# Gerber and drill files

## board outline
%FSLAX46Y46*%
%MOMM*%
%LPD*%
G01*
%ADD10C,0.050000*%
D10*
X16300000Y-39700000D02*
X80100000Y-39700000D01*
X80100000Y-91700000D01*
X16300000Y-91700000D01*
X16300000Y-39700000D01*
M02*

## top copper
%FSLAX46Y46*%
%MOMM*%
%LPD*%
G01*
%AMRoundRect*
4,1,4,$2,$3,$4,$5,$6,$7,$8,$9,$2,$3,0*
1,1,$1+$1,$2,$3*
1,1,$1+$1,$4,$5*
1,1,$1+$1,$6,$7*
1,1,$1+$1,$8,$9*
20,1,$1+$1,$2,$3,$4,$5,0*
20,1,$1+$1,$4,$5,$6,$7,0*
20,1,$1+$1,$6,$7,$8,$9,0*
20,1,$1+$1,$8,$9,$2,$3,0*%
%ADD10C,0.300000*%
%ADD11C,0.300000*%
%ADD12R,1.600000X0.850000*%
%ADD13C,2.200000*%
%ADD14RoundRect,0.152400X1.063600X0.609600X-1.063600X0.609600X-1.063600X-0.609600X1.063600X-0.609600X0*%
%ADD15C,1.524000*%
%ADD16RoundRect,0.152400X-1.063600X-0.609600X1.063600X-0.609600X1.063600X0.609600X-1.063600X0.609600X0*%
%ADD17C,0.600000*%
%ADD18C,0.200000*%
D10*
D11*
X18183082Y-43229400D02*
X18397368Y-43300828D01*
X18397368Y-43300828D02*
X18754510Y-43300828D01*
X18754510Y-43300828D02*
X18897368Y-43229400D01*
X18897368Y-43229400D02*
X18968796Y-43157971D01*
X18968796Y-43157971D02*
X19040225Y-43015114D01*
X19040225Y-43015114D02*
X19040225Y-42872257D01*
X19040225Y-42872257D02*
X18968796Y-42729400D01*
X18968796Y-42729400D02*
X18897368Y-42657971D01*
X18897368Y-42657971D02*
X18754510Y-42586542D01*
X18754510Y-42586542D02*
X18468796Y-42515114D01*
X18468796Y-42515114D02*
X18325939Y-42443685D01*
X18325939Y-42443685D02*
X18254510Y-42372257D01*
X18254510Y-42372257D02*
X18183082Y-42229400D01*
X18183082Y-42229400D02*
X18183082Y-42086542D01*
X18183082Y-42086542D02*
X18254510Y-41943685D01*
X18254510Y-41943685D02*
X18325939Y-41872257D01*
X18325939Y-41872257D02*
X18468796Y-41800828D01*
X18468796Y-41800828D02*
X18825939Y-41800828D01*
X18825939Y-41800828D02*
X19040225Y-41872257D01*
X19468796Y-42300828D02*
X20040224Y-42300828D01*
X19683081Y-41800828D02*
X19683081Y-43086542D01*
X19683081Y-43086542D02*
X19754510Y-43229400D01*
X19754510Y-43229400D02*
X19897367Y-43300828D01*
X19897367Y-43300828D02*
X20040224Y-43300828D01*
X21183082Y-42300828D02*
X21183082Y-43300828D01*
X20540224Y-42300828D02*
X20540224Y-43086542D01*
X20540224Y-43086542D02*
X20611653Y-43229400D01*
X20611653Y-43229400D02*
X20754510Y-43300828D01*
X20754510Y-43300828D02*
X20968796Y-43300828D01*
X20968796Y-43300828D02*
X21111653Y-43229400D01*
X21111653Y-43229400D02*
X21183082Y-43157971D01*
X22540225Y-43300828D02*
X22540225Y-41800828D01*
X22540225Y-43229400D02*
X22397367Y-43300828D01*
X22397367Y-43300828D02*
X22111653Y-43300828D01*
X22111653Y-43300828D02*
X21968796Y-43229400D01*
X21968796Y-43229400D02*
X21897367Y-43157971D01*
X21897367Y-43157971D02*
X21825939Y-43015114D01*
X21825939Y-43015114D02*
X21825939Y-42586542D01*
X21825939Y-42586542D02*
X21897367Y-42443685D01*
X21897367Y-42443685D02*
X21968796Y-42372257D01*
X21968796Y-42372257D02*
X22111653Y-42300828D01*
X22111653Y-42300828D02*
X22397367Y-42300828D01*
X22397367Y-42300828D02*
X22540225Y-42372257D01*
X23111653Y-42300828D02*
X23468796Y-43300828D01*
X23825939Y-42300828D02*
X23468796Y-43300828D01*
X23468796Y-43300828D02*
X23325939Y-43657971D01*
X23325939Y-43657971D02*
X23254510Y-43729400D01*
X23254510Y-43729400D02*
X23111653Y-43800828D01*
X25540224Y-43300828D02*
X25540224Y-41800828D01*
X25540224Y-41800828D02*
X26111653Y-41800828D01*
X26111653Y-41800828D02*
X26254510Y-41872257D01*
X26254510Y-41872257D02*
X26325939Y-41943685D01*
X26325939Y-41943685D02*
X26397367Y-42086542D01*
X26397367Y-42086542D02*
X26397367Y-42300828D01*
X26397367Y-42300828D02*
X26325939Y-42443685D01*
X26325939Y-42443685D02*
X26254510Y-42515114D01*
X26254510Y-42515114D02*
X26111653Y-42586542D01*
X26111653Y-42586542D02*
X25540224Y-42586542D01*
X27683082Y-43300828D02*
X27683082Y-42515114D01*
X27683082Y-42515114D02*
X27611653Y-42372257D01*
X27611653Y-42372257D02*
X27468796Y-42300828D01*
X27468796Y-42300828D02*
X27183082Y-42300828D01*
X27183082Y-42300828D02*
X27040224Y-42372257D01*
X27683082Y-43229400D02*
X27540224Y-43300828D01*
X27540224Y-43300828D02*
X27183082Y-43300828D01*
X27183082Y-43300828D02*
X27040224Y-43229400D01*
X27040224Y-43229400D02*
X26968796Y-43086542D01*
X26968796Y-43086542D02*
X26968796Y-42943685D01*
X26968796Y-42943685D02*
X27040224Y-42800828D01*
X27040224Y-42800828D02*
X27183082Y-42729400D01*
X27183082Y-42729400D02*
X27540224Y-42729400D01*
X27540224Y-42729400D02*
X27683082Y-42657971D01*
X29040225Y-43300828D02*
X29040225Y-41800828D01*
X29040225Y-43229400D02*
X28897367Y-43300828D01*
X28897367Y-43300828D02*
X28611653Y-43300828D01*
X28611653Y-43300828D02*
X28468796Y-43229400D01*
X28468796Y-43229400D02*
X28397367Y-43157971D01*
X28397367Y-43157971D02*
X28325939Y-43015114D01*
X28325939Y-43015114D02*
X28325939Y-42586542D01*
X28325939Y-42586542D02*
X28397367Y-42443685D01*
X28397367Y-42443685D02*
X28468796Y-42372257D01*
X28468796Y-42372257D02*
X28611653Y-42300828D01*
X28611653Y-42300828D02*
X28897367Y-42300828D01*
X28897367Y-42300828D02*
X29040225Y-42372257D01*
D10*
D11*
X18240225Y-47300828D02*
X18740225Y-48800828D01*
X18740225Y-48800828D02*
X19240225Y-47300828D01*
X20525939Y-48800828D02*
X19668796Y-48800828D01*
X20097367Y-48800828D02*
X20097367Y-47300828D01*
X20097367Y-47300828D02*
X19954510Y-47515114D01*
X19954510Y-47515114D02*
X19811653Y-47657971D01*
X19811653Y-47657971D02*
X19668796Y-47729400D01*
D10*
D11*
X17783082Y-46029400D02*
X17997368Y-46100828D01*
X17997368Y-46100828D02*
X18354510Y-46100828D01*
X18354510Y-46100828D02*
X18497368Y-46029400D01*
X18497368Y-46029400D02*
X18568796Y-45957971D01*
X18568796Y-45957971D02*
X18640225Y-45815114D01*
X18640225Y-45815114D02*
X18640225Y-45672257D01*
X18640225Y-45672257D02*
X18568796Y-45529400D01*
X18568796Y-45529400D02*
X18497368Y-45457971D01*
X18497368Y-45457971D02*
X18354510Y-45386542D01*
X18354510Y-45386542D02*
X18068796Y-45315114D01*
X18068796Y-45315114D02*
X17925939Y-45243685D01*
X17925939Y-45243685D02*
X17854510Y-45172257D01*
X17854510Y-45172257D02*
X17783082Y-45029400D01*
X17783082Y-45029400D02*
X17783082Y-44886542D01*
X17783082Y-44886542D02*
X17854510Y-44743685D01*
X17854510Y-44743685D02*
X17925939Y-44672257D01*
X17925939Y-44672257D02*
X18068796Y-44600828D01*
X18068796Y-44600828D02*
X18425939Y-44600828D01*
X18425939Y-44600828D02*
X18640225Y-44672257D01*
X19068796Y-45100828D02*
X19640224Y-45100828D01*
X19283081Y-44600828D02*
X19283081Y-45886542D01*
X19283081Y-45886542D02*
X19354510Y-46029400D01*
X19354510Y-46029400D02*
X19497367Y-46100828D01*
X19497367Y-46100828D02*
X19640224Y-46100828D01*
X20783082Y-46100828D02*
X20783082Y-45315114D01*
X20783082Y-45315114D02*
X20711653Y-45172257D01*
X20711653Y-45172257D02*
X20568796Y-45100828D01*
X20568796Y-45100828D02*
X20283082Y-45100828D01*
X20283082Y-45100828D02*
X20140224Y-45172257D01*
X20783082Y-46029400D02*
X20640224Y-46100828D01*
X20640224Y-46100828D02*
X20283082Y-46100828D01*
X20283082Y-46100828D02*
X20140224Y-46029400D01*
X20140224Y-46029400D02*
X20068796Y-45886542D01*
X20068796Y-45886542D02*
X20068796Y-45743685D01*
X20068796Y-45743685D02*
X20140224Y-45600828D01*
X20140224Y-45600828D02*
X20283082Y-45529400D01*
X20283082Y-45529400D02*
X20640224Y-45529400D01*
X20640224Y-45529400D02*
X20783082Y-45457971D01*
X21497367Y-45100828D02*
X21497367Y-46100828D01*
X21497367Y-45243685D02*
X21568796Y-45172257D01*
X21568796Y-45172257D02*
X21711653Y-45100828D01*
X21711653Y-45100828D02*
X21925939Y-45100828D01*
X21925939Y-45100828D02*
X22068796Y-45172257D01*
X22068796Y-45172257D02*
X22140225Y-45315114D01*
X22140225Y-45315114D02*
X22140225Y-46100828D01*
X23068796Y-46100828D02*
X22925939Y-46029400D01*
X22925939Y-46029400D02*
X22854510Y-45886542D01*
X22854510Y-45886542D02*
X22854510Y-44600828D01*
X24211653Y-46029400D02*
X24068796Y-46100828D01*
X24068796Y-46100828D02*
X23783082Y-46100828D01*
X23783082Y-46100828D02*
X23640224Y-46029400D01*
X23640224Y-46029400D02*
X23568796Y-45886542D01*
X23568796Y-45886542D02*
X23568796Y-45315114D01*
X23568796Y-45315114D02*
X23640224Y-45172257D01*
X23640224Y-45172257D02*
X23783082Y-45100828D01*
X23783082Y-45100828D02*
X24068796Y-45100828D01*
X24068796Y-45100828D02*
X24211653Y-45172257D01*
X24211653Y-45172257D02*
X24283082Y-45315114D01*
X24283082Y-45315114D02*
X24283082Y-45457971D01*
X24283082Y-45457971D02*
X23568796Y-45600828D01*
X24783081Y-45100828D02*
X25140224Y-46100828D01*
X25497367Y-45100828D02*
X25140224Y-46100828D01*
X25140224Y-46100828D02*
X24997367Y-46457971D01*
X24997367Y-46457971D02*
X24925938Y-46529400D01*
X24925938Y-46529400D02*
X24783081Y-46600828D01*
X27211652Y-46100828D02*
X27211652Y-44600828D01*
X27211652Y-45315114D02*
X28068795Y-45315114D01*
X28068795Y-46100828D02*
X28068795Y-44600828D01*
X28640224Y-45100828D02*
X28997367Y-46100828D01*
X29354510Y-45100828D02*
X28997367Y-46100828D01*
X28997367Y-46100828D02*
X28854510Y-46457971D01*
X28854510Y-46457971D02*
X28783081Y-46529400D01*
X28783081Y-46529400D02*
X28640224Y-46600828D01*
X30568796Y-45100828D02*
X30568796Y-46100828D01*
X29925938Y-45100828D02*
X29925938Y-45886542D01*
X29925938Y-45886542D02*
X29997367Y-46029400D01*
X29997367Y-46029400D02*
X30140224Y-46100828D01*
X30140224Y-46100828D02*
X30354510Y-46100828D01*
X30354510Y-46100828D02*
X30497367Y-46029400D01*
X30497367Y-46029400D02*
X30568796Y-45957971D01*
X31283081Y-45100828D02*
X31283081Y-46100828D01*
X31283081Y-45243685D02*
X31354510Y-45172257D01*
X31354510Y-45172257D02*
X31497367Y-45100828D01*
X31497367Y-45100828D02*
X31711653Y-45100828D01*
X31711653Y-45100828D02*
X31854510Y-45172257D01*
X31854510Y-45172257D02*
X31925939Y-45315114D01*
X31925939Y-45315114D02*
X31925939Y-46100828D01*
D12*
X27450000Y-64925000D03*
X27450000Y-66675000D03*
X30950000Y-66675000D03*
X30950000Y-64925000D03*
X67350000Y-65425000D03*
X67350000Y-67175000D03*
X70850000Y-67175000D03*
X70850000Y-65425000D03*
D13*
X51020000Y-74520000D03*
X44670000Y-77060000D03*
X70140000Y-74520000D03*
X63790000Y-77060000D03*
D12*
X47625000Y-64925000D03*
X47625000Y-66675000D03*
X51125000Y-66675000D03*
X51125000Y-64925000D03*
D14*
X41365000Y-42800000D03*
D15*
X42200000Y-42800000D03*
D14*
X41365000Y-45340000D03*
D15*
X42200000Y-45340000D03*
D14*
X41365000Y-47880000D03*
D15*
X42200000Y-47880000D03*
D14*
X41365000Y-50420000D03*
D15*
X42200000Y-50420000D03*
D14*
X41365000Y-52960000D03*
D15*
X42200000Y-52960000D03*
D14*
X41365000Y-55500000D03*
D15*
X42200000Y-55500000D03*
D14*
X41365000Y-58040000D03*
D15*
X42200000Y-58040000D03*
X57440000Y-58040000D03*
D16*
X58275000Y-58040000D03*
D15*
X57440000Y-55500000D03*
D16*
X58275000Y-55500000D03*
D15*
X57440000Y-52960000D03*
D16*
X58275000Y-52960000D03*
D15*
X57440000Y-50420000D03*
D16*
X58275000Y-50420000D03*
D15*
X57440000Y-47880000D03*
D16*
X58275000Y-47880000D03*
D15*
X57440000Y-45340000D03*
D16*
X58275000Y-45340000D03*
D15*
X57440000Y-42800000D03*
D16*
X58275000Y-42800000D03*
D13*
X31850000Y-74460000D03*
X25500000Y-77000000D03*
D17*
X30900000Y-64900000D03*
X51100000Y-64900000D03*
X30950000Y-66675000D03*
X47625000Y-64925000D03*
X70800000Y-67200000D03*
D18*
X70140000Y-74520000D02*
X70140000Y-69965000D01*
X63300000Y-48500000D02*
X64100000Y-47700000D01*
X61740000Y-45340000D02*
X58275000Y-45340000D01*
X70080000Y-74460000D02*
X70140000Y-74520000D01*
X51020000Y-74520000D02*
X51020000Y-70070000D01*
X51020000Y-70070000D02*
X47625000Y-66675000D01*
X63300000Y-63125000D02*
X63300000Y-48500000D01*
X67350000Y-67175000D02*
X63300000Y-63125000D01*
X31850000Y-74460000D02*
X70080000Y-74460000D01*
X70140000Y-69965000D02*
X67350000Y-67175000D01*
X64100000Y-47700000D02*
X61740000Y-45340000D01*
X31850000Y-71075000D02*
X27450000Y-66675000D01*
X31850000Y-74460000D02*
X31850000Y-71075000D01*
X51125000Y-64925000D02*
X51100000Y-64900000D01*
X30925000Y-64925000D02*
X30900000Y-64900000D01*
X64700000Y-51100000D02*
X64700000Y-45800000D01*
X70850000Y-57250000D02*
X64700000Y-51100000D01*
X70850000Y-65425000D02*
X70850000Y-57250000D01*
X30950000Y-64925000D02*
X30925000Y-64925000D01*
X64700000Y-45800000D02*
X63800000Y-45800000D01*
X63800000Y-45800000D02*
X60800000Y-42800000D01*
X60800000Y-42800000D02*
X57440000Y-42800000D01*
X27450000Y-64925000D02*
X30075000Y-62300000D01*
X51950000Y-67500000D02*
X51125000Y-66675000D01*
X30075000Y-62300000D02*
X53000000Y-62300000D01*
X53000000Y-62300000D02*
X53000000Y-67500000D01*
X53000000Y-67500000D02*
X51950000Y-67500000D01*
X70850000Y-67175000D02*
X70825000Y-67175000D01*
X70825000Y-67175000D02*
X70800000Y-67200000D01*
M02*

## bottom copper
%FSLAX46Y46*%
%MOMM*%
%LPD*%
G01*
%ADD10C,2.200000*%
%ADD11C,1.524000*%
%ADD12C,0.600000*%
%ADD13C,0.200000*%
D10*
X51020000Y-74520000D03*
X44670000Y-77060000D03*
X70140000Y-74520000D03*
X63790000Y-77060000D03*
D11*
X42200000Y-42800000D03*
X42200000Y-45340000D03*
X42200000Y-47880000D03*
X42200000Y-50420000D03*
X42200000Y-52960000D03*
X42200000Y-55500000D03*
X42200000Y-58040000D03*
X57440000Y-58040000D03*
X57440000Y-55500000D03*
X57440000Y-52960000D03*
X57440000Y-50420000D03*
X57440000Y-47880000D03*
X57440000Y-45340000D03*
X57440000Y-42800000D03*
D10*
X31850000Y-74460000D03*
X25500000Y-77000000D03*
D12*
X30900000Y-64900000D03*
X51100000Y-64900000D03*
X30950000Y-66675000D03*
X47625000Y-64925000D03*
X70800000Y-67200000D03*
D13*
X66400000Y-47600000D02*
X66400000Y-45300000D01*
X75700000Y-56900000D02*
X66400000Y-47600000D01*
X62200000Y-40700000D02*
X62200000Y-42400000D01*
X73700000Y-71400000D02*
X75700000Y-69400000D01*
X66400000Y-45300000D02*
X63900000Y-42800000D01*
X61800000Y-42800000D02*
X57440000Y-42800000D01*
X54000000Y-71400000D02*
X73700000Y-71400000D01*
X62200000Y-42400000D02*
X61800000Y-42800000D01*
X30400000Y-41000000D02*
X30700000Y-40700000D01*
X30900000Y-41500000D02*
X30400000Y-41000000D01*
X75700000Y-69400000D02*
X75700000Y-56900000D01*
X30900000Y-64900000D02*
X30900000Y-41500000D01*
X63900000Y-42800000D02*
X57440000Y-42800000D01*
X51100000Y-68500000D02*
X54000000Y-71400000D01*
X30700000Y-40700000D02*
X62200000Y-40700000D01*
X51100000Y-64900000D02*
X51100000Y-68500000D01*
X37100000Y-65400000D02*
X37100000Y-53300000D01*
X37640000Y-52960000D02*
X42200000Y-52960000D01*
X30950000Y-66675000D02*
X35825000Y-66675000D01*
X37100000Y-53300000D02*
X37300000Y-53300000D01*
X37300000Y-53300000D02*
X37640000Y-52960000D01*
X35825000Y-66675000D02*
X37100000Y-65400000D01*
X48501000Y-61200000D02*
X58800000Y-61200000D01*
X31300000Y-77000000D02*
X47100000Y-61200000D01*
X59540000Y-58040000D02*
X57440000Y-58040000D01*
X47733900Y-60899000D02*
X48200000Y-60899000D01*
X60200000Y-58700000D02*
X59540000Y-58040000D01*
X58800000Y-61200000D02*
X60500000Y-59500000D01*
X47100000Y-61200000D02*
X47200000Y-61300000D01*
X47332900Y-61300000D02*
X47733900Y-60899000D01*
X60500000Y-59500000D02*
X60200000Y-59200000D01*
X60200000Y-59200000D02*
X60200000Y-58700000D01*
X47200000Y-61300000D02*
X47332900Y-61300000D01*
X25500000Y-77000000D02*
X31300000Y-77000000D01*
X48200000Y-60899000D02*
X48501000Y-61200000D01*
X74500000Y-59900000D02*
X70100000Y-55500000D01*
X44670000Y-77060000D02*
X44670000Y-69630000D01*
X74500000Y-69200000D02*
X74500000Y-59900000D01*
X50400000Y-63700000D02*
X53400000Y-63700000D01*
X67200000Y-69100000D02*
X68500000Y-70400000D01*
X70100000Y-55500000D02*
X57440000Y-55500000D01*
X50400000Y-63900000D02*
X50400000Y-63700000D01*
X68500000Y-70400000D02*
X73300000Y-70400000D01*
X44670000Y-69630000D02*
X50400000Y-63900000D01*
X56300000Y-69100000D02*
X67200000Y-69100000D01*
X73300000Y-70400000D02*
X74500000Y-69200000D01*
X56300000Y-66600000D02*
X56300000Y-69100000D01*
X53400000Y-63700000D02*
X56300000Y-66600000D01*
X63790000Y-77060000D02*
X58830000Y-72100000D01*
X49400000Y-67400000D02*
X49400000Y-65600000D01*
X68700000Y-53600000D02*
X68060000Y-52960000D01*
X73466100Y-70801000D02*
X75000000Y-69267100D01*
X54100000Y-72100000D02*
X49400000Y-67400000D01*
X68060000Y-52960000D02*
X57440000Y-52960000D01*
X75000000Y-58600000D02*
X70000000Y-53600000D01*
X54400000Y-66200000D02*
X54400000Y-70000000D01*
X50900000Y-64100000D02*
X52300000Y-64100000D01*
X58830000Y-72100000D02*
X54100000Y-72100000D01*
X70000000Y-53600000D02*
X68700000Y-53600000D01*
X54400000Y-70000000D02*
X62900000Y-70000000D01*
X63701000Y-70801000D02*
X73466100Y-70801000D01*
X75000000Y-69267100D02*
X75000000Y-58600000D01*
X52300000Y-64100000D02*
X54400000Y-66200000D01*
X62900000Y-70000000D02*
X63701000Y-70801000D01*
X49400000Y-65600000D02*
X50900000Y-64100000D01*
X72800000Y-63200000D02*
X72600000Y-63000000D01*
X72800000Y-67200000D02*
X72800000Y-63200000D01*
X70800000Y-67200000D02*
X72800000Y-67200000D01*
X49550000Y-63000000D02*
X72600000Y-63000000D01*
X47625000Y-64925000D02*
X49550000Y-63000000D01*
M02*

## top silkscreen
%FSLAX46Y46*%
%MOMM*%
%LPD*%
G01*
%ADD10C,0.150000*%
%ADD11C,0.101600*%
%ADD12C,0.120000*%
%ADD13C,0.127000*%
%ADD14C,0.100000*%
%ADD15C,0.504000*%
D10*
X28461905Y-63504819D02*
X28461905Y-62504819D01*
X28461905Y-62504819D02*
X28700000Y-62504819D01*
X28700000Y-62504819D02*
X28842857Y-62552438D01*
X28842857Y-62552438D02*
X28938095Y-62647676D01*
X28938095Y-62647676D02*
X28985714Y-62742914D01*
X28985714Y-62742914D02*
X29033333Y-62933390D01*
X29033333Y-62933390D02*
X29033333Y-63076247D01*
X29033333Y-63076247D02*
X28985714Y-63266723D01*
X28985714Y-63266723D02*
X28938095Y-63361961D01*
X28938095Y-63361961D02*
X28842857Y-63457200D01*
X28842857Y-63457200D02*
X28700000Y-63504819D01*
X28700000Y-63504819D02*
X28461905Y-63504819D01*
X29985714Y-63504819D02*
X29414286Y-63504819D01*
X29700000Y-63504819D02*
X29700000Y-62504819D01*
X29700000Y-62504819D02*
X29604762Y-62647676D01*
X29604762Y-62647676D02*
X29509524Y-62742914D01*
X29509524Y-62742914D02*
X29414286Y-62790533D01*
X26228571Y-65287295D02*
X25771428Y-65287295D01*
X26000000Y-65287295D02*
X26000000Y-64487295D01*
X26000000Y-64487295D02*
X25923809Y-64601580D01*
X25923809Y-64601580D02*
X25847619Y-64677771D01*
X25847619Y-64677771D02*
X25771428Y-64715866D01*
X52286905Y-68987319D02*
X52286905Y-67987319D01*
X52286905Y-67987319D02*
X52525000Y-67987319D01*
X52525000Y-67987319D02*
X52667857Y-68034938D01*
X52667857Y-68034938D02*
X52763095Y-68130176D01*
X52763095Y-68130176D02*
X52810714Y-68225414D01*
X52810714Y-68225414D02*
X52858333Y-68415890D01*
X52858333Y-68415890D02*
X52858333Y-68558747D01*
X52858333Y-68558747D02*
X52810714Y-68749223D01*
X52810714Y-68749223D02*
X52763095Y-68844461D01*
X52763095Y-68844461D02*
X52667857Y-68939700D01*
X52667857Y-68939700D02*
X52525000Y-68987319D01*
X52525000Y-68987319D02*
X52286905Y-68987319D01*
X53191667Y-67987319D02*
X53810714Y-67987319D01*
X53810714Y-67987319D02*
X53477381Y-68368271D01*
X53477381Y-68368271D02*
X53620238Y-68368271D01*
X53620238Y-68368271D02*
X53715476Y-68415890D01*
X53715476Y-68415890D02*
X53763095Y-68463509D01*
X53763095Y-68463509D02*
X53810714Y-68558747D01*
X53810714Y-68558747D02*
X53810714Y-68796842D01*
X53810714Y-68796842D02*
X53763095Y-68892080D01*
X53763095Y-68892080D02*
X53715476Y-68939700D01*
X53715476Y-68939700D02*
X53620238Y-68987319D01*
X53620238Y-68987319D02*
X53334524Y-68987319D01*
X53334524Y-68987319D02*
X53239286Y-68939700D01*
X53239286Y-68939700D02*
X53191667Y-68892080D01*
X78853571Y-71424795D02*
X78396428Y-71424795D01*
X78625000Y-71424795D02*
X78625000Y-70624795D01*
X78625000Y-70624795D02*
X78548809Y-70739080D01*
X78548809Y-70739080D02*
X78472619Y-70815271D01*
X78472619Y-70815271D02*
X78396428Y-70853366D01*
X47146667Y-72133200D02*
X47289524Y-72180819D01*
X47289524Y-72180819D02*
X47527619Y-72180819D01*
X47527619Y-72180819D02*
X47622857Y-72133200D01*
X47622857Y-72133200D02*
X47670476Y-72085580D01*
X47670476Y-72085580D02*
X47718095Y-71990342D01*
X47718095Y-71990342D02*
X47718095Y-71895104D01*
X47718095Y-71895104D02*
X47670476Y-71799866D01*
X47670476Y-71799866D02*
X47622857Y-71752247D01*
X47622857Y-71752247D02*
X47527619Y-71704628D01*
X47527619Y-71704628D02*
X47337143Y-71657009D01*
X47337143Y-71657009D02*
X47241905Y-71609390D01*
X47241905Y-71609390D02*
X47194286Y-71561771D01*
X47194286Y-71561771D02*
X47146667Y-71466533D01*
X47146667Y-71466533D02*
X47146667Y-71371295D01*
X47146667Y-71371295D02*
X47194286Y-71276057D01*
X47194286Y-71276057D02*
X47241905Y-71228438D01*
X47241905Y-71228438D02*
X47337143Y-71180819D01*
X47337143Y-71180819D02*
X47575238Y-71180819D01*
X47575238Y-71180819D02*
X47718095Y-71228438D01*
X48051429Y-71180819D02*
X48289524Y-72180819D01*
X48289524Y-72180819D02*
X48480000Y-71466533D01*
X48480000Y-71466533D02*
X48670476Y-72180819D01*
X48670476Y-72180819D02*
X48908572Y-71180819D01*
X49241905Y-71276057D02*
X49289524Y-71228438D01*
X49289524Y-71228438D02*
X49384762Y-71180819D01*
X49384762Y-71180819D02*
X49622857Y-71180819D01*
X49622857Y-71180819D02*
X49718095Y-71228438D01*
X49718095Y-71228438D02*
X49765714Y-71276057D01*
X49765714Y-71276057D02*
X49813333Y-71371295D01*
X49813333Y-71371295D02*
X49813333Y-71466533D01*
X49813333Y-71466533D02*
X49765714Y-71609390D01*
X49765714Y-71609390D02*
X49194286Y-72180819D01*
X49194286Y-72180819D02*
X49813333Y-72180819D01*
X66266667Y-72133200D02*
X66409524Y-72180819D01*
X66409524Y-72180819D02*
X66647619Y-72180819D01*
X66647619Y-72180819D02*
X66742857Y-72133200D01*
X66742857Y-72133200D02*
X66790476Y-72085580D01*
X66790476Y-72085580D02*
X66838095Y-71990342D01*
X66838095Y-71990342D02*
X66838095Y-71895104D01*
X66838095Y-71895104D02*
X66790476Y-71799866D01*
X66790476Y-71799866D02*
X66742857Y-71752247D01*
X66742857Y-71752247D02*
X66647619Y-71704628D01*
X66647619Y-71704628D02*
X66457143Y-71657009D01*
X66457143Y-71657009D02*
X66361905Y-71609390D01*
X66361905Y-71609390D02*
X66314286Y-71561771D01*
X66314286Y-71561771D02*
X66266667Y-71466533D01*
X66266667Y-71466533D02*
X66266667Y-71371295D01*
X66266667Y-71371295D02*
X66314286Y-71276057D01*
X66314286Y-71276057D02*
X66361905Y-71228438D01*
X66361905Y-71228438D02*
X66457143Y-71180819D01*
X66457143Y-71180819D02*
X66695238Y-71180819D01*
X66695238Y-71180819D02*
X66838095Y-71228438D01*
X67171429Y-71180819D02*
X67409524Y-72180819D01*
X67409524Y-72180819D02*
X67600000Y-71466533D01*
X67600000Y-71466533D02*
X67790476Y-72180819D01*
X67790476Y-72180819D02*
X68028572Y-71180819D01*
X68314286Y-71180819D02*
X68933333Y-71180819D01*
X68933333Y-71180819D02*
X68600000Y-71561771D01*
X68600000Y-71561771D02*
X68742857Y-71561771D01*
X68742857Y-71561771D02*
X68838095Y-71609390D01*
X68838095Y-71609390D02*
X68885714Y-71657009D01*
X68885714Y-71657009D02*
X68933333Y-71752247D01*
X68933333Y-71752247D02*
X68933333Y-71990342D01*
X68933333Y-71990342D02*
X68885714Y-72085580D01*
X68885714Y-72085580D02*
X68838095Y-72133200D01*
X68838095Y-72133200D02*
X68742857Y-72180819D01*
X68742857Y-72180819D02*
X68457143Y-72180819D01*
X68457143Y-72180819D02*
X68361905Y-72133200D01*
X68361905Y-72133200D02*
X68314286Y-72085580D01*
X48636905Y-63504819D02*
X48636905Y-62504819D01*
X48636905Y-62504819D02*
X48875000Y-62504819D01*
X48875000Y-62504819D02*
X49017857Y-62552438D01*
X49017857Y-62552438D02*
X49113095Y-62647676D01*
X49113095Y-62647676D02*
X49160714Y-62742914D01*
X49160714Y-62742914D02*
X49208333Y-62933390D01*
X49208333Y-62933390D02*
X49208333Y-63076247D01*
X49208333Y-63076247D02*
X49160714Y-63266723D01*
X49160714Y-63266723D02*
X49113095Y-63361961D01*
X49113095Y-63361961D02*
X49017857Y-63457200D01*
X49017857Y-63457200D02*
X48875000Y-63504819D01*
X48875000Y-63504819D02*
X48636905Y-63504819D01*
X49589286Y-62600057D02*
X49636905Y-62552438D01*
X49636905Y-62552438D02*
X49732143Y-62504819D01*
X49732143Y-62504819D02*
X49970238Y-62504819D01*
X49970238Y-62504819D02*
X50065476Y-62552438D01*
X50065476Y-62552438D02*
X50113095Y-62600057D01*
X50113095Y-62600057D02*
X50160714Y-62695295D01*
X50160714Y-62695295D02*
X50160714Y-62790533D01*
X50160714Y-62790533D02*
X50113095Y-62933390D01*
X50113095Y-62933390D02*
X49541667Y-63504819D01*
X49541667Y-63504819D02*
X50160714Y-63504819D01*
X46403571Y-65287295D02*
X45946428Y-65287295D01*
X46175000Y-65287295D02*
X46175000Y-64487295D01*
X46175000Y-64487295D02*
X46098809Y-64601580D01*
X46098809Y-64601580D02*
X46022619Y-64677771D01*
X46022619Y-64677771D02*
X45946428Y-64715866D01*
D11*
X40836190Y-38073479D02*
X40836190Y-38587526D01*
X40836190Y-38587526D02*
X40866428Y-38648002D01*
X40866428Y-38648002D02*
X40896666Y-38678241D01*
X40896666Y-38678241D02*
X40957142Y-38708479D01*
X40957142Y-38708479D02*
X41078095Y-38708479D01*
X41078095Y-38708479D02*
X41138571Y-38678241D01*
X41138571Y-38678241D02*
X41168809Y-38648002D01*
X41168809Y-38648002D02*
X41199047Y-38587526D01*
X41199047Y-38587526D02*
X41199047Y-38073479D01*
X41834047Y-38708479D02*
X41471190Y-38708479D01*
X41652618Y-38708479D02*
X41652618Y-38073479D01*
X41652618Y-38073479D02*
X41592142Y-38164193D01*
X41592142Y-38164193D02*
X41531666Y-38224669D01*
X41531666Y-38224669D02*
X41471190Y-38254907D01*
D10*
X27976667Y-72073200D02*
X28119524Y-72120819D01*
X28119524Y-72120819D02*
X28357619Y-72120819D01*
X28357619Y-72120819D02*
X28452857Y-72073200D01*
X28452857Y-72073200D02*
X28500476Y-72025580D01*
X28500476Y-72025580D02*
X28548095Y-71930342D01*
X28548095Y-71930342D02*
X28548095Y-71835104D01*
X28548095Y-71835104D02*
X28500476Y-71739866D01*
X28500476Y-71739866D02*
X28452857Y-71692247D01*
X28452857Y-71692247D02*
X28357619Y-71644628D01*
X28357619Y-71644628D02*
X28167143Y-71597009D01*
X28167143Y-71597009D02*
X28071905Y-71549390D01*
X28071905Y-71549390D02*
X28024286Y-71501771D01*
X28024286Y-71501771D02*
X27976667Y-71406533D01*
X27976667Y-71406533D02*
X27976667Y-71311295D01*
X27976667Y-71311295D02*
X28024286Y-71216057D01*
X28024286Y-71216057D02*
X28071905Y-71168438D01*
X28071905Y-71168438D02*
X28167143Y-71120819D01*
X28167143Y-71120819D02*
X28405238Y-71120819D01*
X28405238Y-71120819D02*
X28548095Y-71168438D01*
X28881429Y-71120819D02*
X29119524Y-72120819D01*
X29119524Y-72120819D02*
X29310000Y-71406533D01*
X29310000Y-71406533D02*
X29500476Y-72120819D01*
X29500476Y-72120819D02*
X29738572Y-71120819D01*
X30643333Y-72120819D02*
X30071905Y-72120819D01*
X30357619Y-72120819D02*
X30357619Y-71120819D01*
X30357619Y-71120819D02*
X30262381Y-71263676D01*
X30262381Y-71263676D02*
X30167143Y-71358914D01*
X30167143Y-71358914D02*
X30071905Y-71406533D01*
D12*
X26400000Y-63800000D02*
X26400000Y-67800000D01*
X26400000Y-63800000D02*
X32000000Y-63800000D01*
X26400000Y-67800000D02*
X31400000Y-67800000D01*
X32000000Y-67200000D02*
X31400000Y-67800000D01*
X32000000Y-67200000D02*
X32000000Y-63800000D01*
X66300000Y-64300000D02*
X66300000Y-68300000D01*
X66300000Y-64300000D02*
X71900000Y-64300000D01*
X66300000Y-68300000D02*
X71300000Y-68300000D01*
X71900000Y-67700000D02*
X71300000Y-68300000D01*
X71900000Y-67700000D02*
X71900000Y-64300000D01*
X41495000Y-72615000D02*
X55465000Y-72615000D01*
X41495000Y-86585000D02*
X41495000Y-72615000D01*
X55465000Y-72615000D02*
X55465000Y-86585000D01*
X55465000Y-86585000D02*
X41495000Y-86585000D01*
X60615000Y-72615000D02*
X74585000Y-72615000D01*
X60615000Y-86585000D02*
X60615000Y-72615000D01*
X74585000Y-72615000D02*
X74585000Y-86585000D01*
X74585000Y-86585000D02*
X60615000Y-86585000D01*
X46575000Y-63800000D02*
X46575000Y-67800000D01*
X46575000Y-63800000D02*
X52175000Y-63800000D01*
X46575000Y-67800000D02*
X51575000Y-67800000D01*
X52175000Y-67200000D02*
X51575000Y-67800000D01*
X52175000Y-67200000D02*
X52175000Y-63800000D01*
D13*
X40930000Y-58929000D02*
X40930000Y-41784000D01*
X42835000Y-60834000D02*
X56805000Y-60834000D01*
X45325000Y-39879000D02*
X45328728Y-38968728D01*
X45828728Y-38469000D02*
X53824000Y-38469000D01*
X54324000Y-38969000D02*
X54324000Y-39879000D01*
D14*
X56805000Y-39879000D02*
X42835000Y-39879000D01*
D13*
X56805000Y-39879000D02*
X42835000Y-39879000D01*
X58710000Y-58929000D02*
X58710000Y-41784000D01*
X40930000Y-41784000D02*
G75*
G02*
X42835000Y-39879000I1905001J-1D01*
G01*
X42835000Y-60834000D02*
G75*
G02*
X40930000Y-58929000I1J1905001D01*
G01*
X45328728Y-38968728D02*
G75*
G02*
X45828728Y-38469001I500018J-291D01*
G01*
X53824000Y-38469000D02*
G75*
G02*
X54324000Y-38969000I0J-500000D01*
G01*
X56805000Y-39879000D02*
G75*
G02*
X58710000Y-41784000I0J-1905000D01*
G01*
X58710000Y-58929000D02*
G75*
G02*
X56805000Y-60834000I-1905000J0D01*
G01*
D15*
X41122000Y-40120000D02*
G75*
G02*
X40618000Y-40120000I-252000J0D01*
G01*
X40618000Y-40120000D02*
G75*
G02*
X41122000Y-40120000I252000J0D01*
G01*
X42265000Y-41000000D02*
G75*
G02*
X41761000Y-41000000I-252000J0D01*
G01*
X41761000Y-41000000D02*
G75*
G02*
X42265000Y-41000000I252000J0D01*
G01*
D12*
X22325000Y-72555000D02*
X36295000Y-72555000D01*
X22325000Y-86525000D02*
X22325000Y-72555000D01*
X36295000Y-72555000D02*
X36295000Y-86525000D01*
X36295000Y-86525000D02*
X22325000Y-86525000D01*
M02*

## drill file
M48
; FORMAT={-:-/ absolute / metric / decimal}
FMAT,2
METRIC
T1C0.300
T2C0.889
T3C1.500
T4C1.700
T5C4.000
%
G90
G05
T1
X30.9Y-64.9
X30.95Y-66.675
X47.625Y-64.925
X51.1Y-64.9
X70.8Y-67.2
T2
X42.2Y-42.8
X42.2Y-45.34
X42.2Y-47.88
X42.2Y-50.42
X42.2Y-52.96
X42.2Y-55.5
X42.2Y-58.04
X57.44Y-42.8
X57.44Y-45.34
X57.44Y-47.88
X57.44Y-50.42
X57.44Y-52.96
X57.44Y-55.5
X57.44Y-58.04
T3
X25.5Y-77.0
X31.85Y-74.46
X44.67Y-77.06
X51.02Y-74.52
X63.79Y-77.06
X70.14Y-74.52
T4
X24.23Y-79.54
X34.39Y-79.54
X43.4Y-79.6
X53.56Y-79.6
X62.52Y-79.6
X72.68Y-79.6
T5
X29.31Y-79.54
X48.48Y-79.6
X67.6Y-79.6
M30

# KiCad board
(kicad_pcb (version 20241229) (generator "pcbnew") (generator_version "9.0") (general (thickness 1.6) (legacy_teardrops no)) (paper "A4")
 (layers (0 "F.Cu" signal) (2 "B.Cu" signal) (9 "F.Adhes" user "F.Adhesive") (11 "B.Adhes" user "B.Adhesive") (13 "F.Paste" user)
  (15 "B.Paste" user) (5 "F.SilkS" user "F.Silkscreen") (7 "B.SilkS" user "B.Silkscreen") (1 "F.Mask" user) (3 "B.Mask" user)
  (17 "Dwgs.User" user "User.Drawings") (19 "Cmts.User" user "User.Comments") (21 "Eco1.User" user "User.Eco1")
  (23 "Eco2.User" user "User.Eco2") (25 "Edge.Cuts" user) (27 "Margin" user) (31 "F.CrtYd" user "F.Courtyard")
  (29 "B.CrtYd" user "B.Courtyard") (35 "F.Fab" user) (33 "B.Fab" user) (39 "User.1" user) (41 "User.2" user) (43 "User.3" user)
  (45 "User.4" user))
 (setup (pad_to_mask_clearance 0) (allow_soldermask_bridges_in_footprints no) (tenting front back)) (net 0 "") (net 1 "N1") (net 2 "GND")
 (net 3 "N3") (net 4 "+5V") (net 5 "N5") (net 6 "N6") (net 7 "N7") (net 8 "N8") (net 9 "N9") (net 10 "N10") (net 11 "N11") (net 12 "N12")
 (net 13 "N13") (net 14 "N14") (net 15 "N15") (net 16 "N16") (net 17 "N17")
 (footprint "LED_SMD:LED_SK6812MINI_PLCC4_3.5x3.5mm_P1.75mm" (layer "F.Cu") (at 29.2 65.8)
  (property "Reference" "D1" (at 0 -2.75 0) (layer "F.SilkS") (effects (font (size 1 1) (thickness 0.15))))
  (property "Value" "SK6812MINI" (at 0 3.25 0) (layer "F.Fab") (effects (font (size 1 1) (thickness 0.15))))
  (fp_line (start -2.8 -2) (end -2.8 2) (stroke (width 0.12) (type default)) (layer "F.SilkS"))
  (fp_line (start -2.8 -2) (end 2.8 -2) (stroke (width 0.12) (type solid)) (layer "F.SilkS"))
  (fp_line (start -2.8 2) (end 2.2 2) (stroke (width 0.12) (type solid)) (layer "F.SilkS"))
  (fp_line (start 2.8 1.4) (end 2.2 2) (stroke (width 0.12) (type default)) (layer "F.SilkS"))
  (fp_line (start 2.8 1.4) (end 2.8 -2) (stroke (width 0.12) (type solid)) (layer "F.SilkS"))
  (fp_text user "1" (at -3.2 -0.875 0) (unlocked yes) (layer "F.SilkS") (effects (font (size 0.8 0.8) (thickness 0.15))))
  (pad "1" smd rect (at -1.75 -0.875) (size 1.6 0.85) (layers "F.Cu" "F.Mask" "F.Paste") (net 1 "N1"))
  (pad "2" smd rect (at -1.75 0.875) (size 1.6 0.85) (layers "F.Cu" "F.Mask" "F.Paste") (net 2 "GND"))
  (pad "3" smd rect (at 1.75 0.875) (size 1.6 0.85) (layers "F.Cu" "F.Mask" "F.Paste") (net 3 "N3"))
  (pad "4" smd rect (at 1.75 -0.875) (size 1.6 0.85) (layers "F.Cu" "F.Mask" "F.Paste") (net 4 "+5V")))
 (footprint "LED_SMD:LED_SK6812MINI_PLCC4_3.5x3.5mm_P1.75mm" (layer "F.Cu") (at 69.1 66.3)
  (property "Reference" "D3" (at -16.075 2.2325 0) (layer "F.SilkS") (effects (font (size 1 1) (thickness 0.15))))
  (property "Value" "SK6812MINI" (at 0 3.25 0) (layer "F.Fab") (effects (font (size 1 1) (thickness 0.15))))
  (fp_line (start -2.8 -2) (end -2.8 2) (stroke (width 0.12) (type default)) (layer "F.SilkS"))
  (fp_line (start -2.8 -2) (end 2.8 -2) (stroke (width 0.12) (type solid)) (layer "F.SilkS"))
  (fp_line (start -2.8 2) (end 2.2 2) (stroke (width 0.12) (type solid)) (layer "F.SilkS"))
  (fp_line (start 2.8 1.4) (end 2.2 2) (stroke (width 0.12) (type default)) (layer "F.SilkS"))
  (fp_line (start 2.8 1.4) (end 2.8 -2) (stroke (width 0.12) (type solid)) (layer "F.SilkS"))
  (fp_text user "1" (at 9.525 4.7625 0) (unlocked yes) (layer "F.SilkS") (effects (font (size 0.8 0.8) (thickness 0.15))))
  (pad "1" smd rect (at -1.75 -0.875) (size 1.6 0.85) (layers "F.Cu" "F.Mask" "F.Paste") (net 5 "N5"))
  (pad "2" smd rect (at -1.75 0.875) (size 1.6 0.85) (layers "F.Cu" "F.Mask" "F.Paste") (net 2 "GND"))
  (pad "3" smd rect (at 1.75 0.875) (size 1.6 0.85) (layers "F.Cu" "F.Mask" "F.Paste") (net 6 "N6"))
  (pad "4" smd rect (at 1.75 -0.875) (size 1.6 0.85) (layers "F.Cu" "F.Mask" "F.Paste") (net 4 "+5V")))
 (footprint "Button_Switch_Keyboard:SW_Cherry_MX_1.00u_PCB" (layer "F.Cu") (at 51.02 74.52)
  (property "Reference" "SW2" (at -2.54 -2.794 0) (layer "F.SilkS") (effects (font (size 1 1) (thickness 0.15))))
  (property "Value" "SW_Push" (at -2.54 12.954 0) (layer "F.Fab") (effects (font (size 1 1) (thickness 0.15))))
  (fp_line (start -9.525 -1.905) (end 4.445 -1.905) (stroke (width 0.12) (type solid)) (layer "F.SilkS"))
  (fp_line (start -9.525 12.065) (end -9.525 -1.905) (stroke (width 0.12) (type solid)) (layer "F.SilkS"))
  (fp_line (start 4.445 -1.905) (end 4.445 12.065) (stroke (width 0.12) (type solid)) (layer "F.SilkS"))
  (fp_line (start 4.445 12.065) (end -9.525 12.065) (stroke (width 0.12) (type solid)) (layer "F.SilkS"))
  (pad "" np_thru_hole circle (at -7.62 5.08) (size 1.7 1.7) (drill 1.7) (layers "*.Cu" "*.Mask"))
  (pad "" np_thru_hole circle (at -2.54 5.08) (size 4 4) (drill 4) (layers "*.Cu" "*.Mask"))
  (pad "" np_thru_hole circle (at 2.54 5.08) (size 1.7 1.7) (drill 1.7) (layers "*.Cu" "*.Mask"))
  (pad "1" thru_hole circle (at 0 0) (size 2.2 2.2) (drill 1.5) (layers "*.Cu" "*.Mask") (remove_unused_layers no) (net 2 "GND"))
  (pad "2" thru_hole circle (at -6.35 2.54) (size 2.2 2.2) (drill 1.5) (layers "*.Cu" "*.Mask") (remove_unused_layers no) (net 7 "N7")))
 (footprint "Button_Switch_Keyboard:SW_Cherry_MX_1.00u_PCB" (layer "F.Cu") (at 70.14 74.52)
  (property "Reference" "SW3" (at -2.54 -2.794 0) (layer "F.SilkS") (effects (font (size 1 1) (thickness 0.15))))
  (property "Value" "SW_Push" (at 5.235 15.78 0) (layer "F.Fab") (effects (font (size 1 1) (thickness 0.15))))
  (fp_line (start -9.525 -1.905) (end 4.445 -1.905) (stroke (width 0.12) (type solid)) (layer "F.SilkS"))
  (fp_line (start -9.525 12.065) (end -9.525 -1.905) (stroke (width 0.12) (type solid)) (layer "F.SilkS"))
  (fp_line (start 4.445 -1.905) (end 4.445 12.065) (stroke (width 0.12) (type solid)) (layer "F.SilkS"))
  (fp_line (start 4.445 12.065) (end -9.525 12.065) (stroke (width 0.12) (type solid)) (layer "F.SilkS"))
  (pad "" np_thru_hole circle (at -7.62 5.08) (size 1.7 1.7) (drill 1.7) (layers "*.Cu" "*.Mask"))
  (pad "" np_thru_hole circle (at -2.54 5.08) (size 4 4) (drill 4) (layers "*.Cu" "*.Mask"))
  (pad "" np_thru_hole circle (at 2.54 5.08) (size 1.7 1.7) (drill 1.7) (layers "*.Cu" "*.Mask"))
  (pad "1" thru_hole circle (at 0 0) (size 2.2 2.2) (drill 1.5) (layers "*.Cu" "*.Mask") (remove_unused_layers no) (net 2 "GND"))
  (pad "2" thru_hole circle (at -6.35 2.54) (size 2.2 2.2) (drill 1.5) (layers "*.Cu" "*.Mask") (remove_unused_layers no) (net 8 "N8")))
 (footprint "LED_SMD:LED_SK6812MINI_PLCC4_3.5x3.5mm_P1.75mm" (layer "F.Cu") (at 49.375 65.8)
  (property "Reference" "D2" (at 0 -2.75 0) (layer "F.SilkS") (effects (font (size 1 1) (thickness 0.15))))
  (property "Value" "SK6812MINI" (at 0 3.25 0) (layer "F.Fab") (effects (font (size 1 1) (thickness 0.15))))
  (fp_line (start -2.8 -2) (end -2.8 2) (stroke (width 0.12) (type default)) (layer "F.SilkS"))
  (fp_line (start -2.8 -2) (end 2.8 -2) (stroke (width 0.12) (type solid)) (layer "F.SilkS"))
  (fp_line (start -2.8 2) (end 2.2 2) (stroke (width 0.12) (type solid)) (layer "F.SilkS"))
  (fp_line (start 2.8 1.4) (end 2.2 2) (stroke (width 0.12) (type default)) (layer "F.SilkS"))
  (fp_line (start 2.8 1.4) (end 2.8 -2) (stroke (width 0.12) (type solid)) (layer "F.SilkS"))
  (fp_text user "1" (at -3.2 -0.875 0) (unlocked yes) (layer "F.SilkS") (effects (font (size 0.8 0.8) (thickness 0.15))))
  (pad "1" smd rect (at -1.75 -0.875) (size 1.6 0.85) (layers "F.Cu" "F.Mask" "F.Paste") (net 6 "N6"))
  (pad "2" smd rect (at -1.75 0.875) (size 1.6 0.85) (layers "F.Cu" "F.Mask" "F.Paste") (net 2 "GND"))
  (pad "3" smd rect (at 1.75 0.875) (size 1.6 0.85) (layers "F.Cu" "F.Mask" "F.Paste") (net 1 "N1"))
  (pad "4" smd rect (at 1.75 -0.875) (size 1.6 0.85) (layers "F.Cu" "F.Mask" "F.Paste") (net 4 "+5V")))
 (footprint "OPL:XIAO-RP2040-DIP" (layer "F.Cu") (at 49.82 50.42)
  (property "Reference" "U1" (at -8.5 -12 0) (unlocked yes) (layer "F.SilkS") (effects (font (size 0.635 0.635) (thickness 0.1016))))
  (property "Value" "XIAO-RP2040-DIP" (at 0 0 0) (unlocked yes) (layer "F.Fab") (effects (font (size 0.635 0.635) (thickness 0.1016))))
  (fp_line (start -8.89 8.509) (end -8.89 -8.636) (stroke (width 0.127) (type solid)) (layer "F.SilkS"))
  (fp_line (start -6.985 10.414) (end 6.985 10.414) (stroke (width 0.127) (type solid)) (layer "F.SilkS"))
  (fp_line (start -4.495 -10.541) (end -4.491272 -11.451272) (stroke (width 0.127) (type solid)) (layer "F.SilkS"))
  (fp_line (start -3.991272 -11.951) (end 4.004 -11.951) (stroke (width 0.127) (type solid)) (layer "F.SilkS"))
  (fp_line (start 4.504 -11.451) (end 4.504 -10.541) (stroke (width 0.127) (type solid)) (layer "F.SilkS"))
  (fp_line (start 6.985 -10.541) (end -6.985 -10.541) (stroke (width 0.1) (type solid)) (layer "F.SilkS"))
  (fp_line (start 6.985 -10.541) (end -6.985 -10.541) (stroke (width 0.127) (type solid)) (layer "F.SilkS"))
  (fp_line (start 8.89 8.509) (end 8.89 -8.636) (stroke (width 0.127) (type solid)) (layer "F.SilkS"))
  (fp_arc (start -8.89 -8.636) (mid -8.332038 -9.983038) (end -6.985 -10.541) (stroke (width 0.127) (type solid)) (layer "F.SilkS"))
  (fp_arc (start -6.985 10.414) (mid -8.332038 9.856038) (end -8.89 8.509) (stroke (width 0.127) (type solid)) (layer "F.SilkS"))
  (fp_arc (start -4.491272 -11.451272) (mid -4.344728 -11.80464) (end -3.991272 -11.951) (stroke (width 0.127) (type default))
   (layer "F.SilkS"))
  (fp_arc (start 4.004 -11.951) (mid 4.357553 -11.804553) (end 4.504 -11.451) (stroke (width 0.127) (type default)) (layer "F.SilkS"))
  (fp_arc (start 6.985 -10.541) (mid 8.332038 -9.983038) (end 8.89 -8.636) (stroke (width 0.127) (type solid)) (layer "F.SilkS"))
  (fp_arc (start 8.89 8.509) (mid 8.332038 9.856038) (end 6.985 10.414) (stroke (width 0.127) (type solid)) (layer "F.SilkS"))
  (fp_circle (center -8.95 -10.3) (end -8.95 -10.554) (stroke (width 0.5) (type solid)) (fill yes) (layer "F.SilkS"))
  (fp_circle (center -7.807 -9.42) (end -7.807 -9.674) (stroke (width 0.5) (type solid)) (fill yes) (layer "F.SilkS"))
  (pad "1" smd roundrect (at -8.455 -7.62 180) (size 2.432 1.524) (layers "F.Cu" "F.Mask") (roundrect_rratio 0.1) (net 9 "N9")
   (thermal_bridge_angle 45))
  (pad "1" thru_hole circle (at -7.62 -7.62 180) (size 1.524 1.524) (drill 0.889) (layers "*.Cu" "*.Mask") (remove_unused_layers no)
   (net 9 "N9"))
  (pad "2" smd roundrect (at -8.455 -5.08 180) (size 2.432 1.524) (layers "F.Cu" "F.Mask") (roundrect_rratio 0.1) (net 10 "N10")
   (thermal_bridge_angle 45))
  (pad "2" thru_hole circle (at -7.62 -5.08 180) (size 1.524 1.524) (drill 0.889) (layers "*.Cu" "*.Mask") (remove_unused_layers no)
   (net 10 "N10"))
  (pad "3" smd roundrect (at -8.455 -2.54 180) (size 2.432 1.524) (layers "F.Cu" "F.Mask") (roundrect_rratio 0.1) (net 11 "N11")
   (thermal_bridge_angle 45))
  (pad "3" thru_hole circle (at -7.62 -2.54 180) (size 1.524 1.524) (drill 0.889) (layers "*.Cu" "*.Mask") (remove_unused_layers no)
   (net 11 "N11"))
  (pad "4" smd roundrect (at -8.455 0 180) (size 2.432 1.524) (layers "F.Cu" "F.Mask") (roundrect_rratio 0.1) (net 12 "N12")
   (thermal_bridge_angle 45))
  (pad "4" thru_hole circle (at -7.62 0 180) (size 1.524 1.524) (drill 0.889) (layers "*.Cu" "*.Mask") (remove_unused_layers no)
   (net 12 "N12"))
  (pad "5" smd roundrect (at -8.455 2.54 180) (size 2.432 1.524) (layers "F.Cu" "F.Mask") (roundrect_rratio 0.1) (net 3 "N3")
   (thermal_bridge_angle 45))
  (pad "5" thru_hole circle (at -7.62 2.54 180) (size 1.524 1.524) (drill 0.889) (layers "*.Cu" "*.Mask") (remove_unused_layers no)
   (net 3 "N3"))
  (pad "6" smd roundrect (at -8.455 5.08 180) (size 2.432 1.524) (layers "F.Cu" "F.Mask") (roundrect_rratio 0.1) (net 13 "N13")
   (thermal_bridge_angle 45))
  (pad "6" thru_hole circle (at -7.62 5.08 180) (size 1.524 1.524) (drill 0.889) (layers "*.Cu" "*.Mask") (remove_unused_layers no)
   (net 13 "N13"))
  (pad "7" smd roundrect (at -8.455 7.62 180) (size 2.432 1.524) (layers "F.Cu" "F.Mask") (roundrect_rratio 0.1) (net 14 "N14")
   (thermal_bridge_angle 45))
  (pad "7" thru_hole circle (at -7.62 7.62 180) (size 1.524 1.524) (drill 0.889) (layers "*.Cu" "*.Mask") (remove_unused_layers no)
   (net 14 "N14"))
  (pad "8" thru_hole circle (at 7.62 7.62) (size 1.524 1.524) (drill 0.889) (layers "*.Cu" "*.Mask") (remove_unused_layers no)
   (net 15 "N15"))
  (pad "8" smd roundrect (at 8.455 7.62) (size 2.432 1.524) (layers "F.Cu" "F.Mask") (roundrect_rratio 0.1) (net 15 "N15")
   (thermal_bridge_angle 45))
  (pad "9" thru_hole circle (at 7.62 5.08) (size 1.524 1.524) (drill 0.889) (layers "*.Cu" "*.Mask") (remove_unused_layers no) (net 7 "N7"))
  (pad "9" smd roundrect (at 8.455 5.08) (size 2.432 1.524) (layers "F.Cu" "F.Mask") (roundrect_rratio 0.1) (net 7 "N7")
   (thermal_bridge_angle 45))
  (pad "10" thru_hole circle (at 7.62 2.54) (size 1.524 1.524) (drill 0.889) (layers "*.Cu" "*.Mask") (remove_unused_layers no) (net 8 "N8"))
  (pad "10" smd roundrect (at 8.455 2.54) (size 2.432 1.524) (layers "F.Cu" "F.Mask") (roundrect_rratio 0.1) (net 8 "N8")
   (thermal_bridge_angle 45))
  (pad "11" thru_hole circle (at 7.62 0) (size 1.524 1.524) (drill 0.889) (layers "*.Cu" "*.Mask") (remove_unused_layers no) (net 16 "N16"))
  (pad "11" smd roundrect (at 8.455 0) (size 2.432 1.524) (layers "F.Cu" "F.Mask") (roundrect_rratio 0.1) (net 16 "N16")
   (thermal_bridge_angle 45))
  (pad "12" thru_hole circle (at 7.62 -2.54) (size 1.524 1.524) (drill 0.889) (layers "*.Cu" "*.Mask") (remove_unused_layers no)
   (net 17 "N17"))
  (pad "12" smd roundrect (at 8.455 -2.54) (size 2.432 1.524) (layers "F.Cu" "F.Mask") (roundrect_rratio 0.1) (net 17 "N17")
   (thermal_bridge_angle 45))
  (pad "13" thru_hole circle (at 7.62 -5.08) (size 1.524 1.524) (drill 0.889) (layers "*.Cu" "*.Mask") (remove_unused_layers no)
   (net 2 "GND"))
  (pad "13" smd roundrect (at 8.455 -5.08) (size 2.432 1.524) (layers "F.Cu" "F.Mask") (roundrect_rratio 0.1) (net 2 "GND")
   (thermal_bridge_angle 45))
  (pad "14" thru_hole circle (at 7.62 -7.62) (size 1.524 1.524) (drill 0.889) (layers "*.Cu" "*.Mask") (remove_unused_layers no)
   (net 4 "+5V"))
  (pad "14" smd roundrect (at 8.455 -7.62) (size 2.432 1.524) (layers "F.Cu" "F.Mask") (roundrect_rratio 0.1) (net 4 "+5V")
   (thermal_bridge_angle 45)))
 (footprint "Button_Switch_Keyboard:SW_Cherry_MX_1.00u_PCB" (layer "F.Cu") (at 31.85 74.46)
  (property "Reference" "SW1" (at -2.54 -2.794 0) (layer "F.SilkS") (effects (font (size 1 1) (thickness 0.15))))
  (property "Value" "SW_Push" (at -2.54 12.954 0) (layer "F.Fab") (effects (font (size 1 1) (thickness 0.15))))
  (fp_line (start -9.525 -1.905) (end 4.445 -1.905) (stroke (width 0.12) (type solid)) (layer "F.SilkS"))
  (fp_line (start -9.525 12.065) (end -9.525 -1.905) (stroke (width 0.12) (type solid)) (layer "F.SilkS"))
  (fp_line (start 4.445 -1.905) (end 4.445 12.065) (stroke (width 0.12) (type solid)) (layer "F.SilkS"))
  (fp_line (start 4.445 12.065) (end -9.525 12.065) (stroke (width 0.12) (type solid)) (layer "F.SilkS"))
  (pad "" np_thru_hole circle (at -7.62 5.08) (size 1.7 1.7) (drill 1.7) (layers "*.Cu" "*.Mask"))
  (pad "" np_thru_hole circle (at -2.54 5.08) (size 4 4) (drill 4) (layers "*.Cu" "*.Mask"))
  (pad "" np_thru_hole circle (at 2.54 5.08) (size 1.7 1.7) (drill 1.7) (layers "*.Cu" "*.Mask"))
  (pad "1" thru_hole circle (at 0 0) (size 2.2 2.2) (drill 1.5) (layers "*.Cu" "*.Mask") (remove_unused_layers no) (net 2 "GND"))
  (pad "2" thru_hole circle (at -6.35 2.54) (size 2.2 2.2) (drill 1.5) (layers "*.Cu" "*.Mask") (remove_unused_layers no) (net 15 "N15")))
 (gr_rect (start 16.3 39.7) (end 80.1 91.7) (stroke (width 0.05) (type default)) (fill no) (layer "Edge.Cuts"))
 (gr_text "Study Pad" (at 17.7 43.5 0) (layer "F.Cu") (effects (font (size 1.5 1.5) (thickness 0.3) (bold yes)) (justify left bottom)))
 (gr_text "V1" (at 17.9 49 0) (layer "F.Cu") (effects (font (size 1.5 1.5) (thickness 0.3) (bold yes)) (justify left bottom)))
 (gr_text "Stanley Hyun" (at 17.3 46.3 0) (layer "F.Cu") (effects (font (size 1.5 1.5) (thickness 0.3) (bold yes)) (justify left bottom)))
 (segment (start 70.14 74.52) (end 70.14 69.965) (width 0.2) (layer "F.Cu") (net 2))
 (segment (start 63.3 48.5) (end 64.1 47.7) (width 0.2) (layer "F.Cu") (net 2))
 (segment (start 61.74 45.34) (end 58.275 45.34) (width 0.2) (layer "F.Cu") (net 2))
 (segment (start 70.08 74.46) (end 70.14 74.52) (width 0.2) (layer "F.Cu") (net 2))
 (segment (start 51.02 74.52) (end 51.02 70.07) (width 0.2) (layer "F.Cu") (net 2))
 (segment (start 51.02 70.07) (end 47.625 66.675) (width 0.2) (layer "F.Cu") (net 2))
 (segment (start 63.3 63.125) (end 63.3 48.5) (width 0.2) (layer "F.Cu") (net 2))
 (segment (start 67.35 67.175) (end 63.3 63.125) (width 0.2) (layer "F.Cu") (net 2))
 (segment (start 31.85 74.46) (end 70.08 74.46) (width 0.2) (layer "F.Cu") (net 2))
 (segment (start 70.14 69.965) (end 67.35 67.175) (width 0.2) (layer "F.Cu") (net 2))
 (segment (start 64.1 47.7) (end 61.74 45.34) (width 0.2) (layer "F.Cu") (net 2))
 (segment (start 31.85 71.075) (end 27.45 66.675) (width 0.2) (layer "F.Cu") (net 2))
 (segment (start 31.85 74.46) (end 31.85 71.075) (width 0.2) (layer "F.Cu") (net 2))
 (segment (start 51.125 64.925) (end 51.1 64.9) (width 0.2) (layer "F.Cu") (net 4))
 (segment (start 30.925 64.925) (end 30.9 64.9) (width 0.2) (layer "F.Cu") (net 4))
 (segment (start 64.7 51.1) (end 64.7 45.8) (width 0.2) (layer "F.Cu") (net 4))
 (segment (start 70.85 57.25) (end 64.7 51.1) (width 0.2) (layer "F.Cu") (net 4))
 (segment (start 70.85 65.425) (end 70.85 57.25) (width 0.2) (layer "F.Cu") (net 4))
 (segment (start 30.95 64.925) (end 30.925 64.925) (width 0.2) (layer "F.Cu") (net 4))
 (segment (start 64.7 45.8) (end 63.8 45.8) (width 0.2) (layer "F.Cu") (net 4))
 (segment (start 63.8 45.8) (end 60.8 42.8) (width 0.2) (layer "F.Cu") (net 4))
 (segment (start 60.8 42.8) (end 57.44 42.8) (width 0.2) (layer "F.Cu") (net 4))
 (via (at 30.9 64.9) (size 0.6) (drill 0.3) (layers "F.Cu" "B.Cu") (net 4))
 (via (at 51.1 64.9) (size 0.6) (drill 0.3) (layers "F.Cu" "B.Cu") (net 4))
 (segment (start 66.4 47.6) (end 66.4 45.3) (width 0.2) (layer "B.Cu") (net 4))
 (segment (start 75.7 56.9) (end 66.4 47.6) (width 0.2) (layer "B.Cu") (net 4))
 (segment (start 62.2 40.7) (end 62.2 42.4) (width 0.2) (layer "B.Cu") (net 4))
 (segment (start 73.7 71.4) (end 75.7 69.4) (width 0.2) (layer "B.Cu") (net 4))
 (segment (start 66.4 45.3) (end 63.9 42.8) (width 0.2) (layer "B.Cu") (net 4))
 (segment (start 61.8 42.8) (end 57.44 42.8) (width 0.2) (layer "B.Cu") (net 4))
 (segment (start 54 71.4) (end 73.7 71.4) (width 0.2) (layer "B.Cu") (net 4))
 (segment (start 62.2 42.4) (end 61.8 42.8) (width 0.2) (layer "B.Cu") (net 4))
 (segment (start 30.4 41) (end 30.7 40.7) (width 0.2) (layer "B.Cu") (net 4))
 (segment (start 30.9 41.5) (end 30.4 41) (width 0.2) (layer "B.Cu") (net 4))
 (segment (start 75.7 69.4) (end 75.7 56.9) (width 0.2) (layer "B.Cu") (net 4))
 (segment (start 30.9 64.9) (end 30.9 41.5) (width 0.2) (layer "B.Cu") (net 4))
 (segment (start 63.9 42.8) (end 57.44 42.8) (width 0.2) (layer "B.Cu") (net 4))
 (segment (start 51.1 68.5) (end 54 71.4) (width 0.2) (layer "B.Cu") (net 4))
 (segment (start 30.7 40.7) (end 62.2 40.7) (width 0.2) (layer "B.Cu") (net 4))
 (segment (start 51.1 64.9) (end 51.1 68.5) (width 0.2) (layer "B.Cu") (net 4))
 (via (at 30.95 66.675) (size 0.6) (drill 0.3) (layers "F.Cu" "B.Cu") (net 3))
 (segment (start 37.1 65.4) (end 37.1 53.3) (width 0.2) (layer "B.Cu") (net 3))
 (segment (start 37.64 52.96) (end 42.2 52.96) (width 0.2) (layer "B.Cu") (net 3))
 (segment (start 30.95 66.675) (end 35.825 66.675) (width 0.2) (layer "B.Cu") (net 3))
 (segment (start 37.1 53.3) (end 37.3 53.3) (width 0.2) (layer "B.Cu") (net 3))
 (segment (start 37.3 53.3) (end 37.64 52.96) (width 0.2) (layer "B.Cu") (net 3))
 (segment (start 35.825 66.675) (end 37.1 65.4) (width 0.2) (layer "B.Cu") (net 3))
 (segment (start 48.501 61.2) (end 58.8 61.2) (width 0.2) (layer "B.Cu") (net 15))
 (segment (start 31.3 77) (end 47.1 61.2) (width 0.2) (layer "B.Cu") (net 15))
 (segment (start 59.54 58.04) (end 57.44 58.04) (width 0.2) (layer "B.Cu") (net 15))
 (segment (start 47.7339 60.899) (end 48.2 60.899) (width 0.2) (layer "B.Cu") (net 15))
 (segment (start 60.2 58.7) (end 59.54 58.04) (width 0.2) (layer "B.Cu") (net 15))
 (segment (start 58.8 61.2) (end 60.5 59.5) (width 0.2) (layer "B.Cu") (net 15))
 (segment (start 47.1 61.2) (end 47.2 61.3) (width 0.2) (layer "B.Cu") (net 15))
 (segment (start 47.3329 61.3) (end 47.7339 60.899) (width 0.2) (layer "B.Cu") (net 15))
 (segment (start 60.5 59.5) (end 60.2 59.2) (width 0.2) (layer "B.Cu") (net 15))
 (segment (start 60.2 59.2) (end 60.2 58.7) (width 0.2) (layer "B.Cu") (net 15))
 (segment (start 47.2 61.3) (end 47.3329 61.3) (width 0.2) (layer "B.Cu") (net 15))
 (segment (start 25.5 77) (end 31.3 77) (width 0.2) (layer "B.Cu") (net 15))
 (segment (start 48.2 60.899) (end 48.501 61.2) (width 0.2) (layer "B.Cu") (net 15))
 (segment (start 74.5 59.9) (end 70.1 55.5) (width 0.2) (layer "B.Cu") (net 7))
 (segment (start 44.67 77.06) (end 44.67 69.63) (width 0.2) (layer "B.Cu") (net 7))
 (segment (start 74.5 69.2) (end 74.5 59.9) (width 0.2) (layer "B.Cu") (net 7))
 (segment (start 50.4 63.7) (end 53.4 63.7) (width 0.2) (layer "B.Cu") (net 7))
 (segment (start 67.2 69.1) (end 68.5 70.4) (width 0.2) (layer "B.Cu") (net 7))
 (segment (start 70.1 55.5) (end 57.44 55.5) (width 0.2) (layer "B.Cu") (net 7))
 (segment (start 50.4 63.9) (end 50.4 63.7) (width 0.2) (layer "B.Cu") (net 7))
 (segment (start 68.5 70.4) (end 73.3 70.4) (width 0.2) (layer "B.Cu") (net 7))
 (segment (start 44.67 69.63) (end 50.4 63.9) (width 0.2) (layer "B.Cu") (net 7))
 (segment (start 56.3 69.1) (end 67.2 69.1) (width 0.2) (layer "B.Cu") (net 7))
 (segment (start 73.3 70.4) (end 74.5 69.2) (width 0.2) (layer "B.Cu") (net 7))
 (segment (start 56.3 66.6) (end 56.3 69.1) (width 0.2) (layer "B.Cu") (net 7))
 (segment (start 53.4 63.7) (end 56.3 66.6) (width 0.2) (layer "B.Cu") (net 7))
 (segment (start 63.79 77.06) (end 58.83 72.1) (width 0.2) (layer "B.Cu") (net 8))
 (segment (start 49.4 67.4) (end 49.4 65.6) (width 0.2) (layer "B.Cu") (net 8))
 (segment (start 68.7 53.6) (end 68.06 52.96) (width 0.2) (layer "B.Cu") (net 8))
 (segment (start 73.4661 70.801) (end 75 69.2671) (width 0.2) (layer "B.Cu") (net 8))
 (segment (start 54.1 72.1) (end 49.4 67.4) (width 0.2) (layer "B.Cu") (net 8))
 (segment (start 68.06 52.96) (end 57.44 52.96) (width 0.2) (layer "B.Cu") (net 8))
 (segment (start 75 58.6) (end 70 53.6) (width 0.2) (layer "B.Cu") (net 8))
 (segment (start 54.4 66.2) (end 54.4 70) (width 0.2) (layer "B.Cu") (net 8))
 (segment (start 50.9 64.1) (end 52.3 64.1) (width 0.2) (layer "B.Cu") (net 8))
 (segment (start 58.83 72.1) (end 54.1 72.1) (width 0.2) (layer "B.Cu") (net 8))
 (segment (start 70 53.6) (end 68.7 53.6) (width 0.2) (layer "B.Cu") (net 8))
 (segment (start 54.4 70) (end 62.9 70) (width 0.2) (layer "B.Cu") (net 8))
 (segment (start 63.701 70.801) (end 73.4661 70.801) (width 0.2) (layer "B.Cu") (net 8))
 (segment (start 75 69.2671) (end 75 58.6) (width 0.2) (layer "B.Cu") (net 8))
 (segment (start 52.3 64.1) (end 54.4 66.2) (width 0.2) (layer "B.Cu") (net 8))
 (segment (start 62.9 70) (end 63.701 70.801) (width 0.2) (layer "B.Cu") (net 8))
 (segment (start 49.4 65.6) (end 50.9 64.1) (width 0.2) (layer "B.Cu") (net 8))
 (segment (start 27.45 64.925) (end 30.075 62.3) (width 0.2) (layer "F.Cu") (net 1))
 (segment (start 51.95 67.5) (end 51.125 66.675) (width 0.2) (layer "F.Cu") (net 1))
 (segment (start 30.075 62.3) (end 53 62.3) (width 0.2) (layer "F.Cu") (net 1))
 (segment (start 53 62.3) (end 53 67.5) (width 0.2) (layer "F.Cu") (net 1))
 (segment (start 53 67.5) (end 51.95 67.5) (width 0.2) (layer "F.Cu") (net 1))
 (segment (start 70.85 67.175) (end 70.825 67.175) (width 0.2) (layer "F.Cu") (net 6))
 (segment (start 70.825 67.175) (end 70.8 67.2) (width 0.2) (layer "F.Cu") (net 6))
 (via (at 47.625 64.925) (size 0.6) (drill 0.3) (layers "F.Cu" "B.Cu") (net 6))
 (via (at 70.8 67.2) (size 0.6) (drill 0.3) (layers "F.Cu" "B.Cu") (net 6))
 (segment (start 72.8 63.2) (end 72.6 63) (width 0.2) (layer "B.Cu") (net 6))
 (segment (start 72.8 67.2) (end 72.8 63.2) (width 0.2) (layer "B.Cu") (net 6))
 (segment (start 70.8 67.2) (end 72.8 67.2) (width 0.2) (layer "B.Cu") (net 6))
 (segment (start 49.55 63) (end 72.6 63) (width 0.2) (layer "B.Cu") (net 6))
 (segment (start 47.625 64.925) (end 49.55 63) (width 0.2) (layer "B.Cu") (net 6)))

